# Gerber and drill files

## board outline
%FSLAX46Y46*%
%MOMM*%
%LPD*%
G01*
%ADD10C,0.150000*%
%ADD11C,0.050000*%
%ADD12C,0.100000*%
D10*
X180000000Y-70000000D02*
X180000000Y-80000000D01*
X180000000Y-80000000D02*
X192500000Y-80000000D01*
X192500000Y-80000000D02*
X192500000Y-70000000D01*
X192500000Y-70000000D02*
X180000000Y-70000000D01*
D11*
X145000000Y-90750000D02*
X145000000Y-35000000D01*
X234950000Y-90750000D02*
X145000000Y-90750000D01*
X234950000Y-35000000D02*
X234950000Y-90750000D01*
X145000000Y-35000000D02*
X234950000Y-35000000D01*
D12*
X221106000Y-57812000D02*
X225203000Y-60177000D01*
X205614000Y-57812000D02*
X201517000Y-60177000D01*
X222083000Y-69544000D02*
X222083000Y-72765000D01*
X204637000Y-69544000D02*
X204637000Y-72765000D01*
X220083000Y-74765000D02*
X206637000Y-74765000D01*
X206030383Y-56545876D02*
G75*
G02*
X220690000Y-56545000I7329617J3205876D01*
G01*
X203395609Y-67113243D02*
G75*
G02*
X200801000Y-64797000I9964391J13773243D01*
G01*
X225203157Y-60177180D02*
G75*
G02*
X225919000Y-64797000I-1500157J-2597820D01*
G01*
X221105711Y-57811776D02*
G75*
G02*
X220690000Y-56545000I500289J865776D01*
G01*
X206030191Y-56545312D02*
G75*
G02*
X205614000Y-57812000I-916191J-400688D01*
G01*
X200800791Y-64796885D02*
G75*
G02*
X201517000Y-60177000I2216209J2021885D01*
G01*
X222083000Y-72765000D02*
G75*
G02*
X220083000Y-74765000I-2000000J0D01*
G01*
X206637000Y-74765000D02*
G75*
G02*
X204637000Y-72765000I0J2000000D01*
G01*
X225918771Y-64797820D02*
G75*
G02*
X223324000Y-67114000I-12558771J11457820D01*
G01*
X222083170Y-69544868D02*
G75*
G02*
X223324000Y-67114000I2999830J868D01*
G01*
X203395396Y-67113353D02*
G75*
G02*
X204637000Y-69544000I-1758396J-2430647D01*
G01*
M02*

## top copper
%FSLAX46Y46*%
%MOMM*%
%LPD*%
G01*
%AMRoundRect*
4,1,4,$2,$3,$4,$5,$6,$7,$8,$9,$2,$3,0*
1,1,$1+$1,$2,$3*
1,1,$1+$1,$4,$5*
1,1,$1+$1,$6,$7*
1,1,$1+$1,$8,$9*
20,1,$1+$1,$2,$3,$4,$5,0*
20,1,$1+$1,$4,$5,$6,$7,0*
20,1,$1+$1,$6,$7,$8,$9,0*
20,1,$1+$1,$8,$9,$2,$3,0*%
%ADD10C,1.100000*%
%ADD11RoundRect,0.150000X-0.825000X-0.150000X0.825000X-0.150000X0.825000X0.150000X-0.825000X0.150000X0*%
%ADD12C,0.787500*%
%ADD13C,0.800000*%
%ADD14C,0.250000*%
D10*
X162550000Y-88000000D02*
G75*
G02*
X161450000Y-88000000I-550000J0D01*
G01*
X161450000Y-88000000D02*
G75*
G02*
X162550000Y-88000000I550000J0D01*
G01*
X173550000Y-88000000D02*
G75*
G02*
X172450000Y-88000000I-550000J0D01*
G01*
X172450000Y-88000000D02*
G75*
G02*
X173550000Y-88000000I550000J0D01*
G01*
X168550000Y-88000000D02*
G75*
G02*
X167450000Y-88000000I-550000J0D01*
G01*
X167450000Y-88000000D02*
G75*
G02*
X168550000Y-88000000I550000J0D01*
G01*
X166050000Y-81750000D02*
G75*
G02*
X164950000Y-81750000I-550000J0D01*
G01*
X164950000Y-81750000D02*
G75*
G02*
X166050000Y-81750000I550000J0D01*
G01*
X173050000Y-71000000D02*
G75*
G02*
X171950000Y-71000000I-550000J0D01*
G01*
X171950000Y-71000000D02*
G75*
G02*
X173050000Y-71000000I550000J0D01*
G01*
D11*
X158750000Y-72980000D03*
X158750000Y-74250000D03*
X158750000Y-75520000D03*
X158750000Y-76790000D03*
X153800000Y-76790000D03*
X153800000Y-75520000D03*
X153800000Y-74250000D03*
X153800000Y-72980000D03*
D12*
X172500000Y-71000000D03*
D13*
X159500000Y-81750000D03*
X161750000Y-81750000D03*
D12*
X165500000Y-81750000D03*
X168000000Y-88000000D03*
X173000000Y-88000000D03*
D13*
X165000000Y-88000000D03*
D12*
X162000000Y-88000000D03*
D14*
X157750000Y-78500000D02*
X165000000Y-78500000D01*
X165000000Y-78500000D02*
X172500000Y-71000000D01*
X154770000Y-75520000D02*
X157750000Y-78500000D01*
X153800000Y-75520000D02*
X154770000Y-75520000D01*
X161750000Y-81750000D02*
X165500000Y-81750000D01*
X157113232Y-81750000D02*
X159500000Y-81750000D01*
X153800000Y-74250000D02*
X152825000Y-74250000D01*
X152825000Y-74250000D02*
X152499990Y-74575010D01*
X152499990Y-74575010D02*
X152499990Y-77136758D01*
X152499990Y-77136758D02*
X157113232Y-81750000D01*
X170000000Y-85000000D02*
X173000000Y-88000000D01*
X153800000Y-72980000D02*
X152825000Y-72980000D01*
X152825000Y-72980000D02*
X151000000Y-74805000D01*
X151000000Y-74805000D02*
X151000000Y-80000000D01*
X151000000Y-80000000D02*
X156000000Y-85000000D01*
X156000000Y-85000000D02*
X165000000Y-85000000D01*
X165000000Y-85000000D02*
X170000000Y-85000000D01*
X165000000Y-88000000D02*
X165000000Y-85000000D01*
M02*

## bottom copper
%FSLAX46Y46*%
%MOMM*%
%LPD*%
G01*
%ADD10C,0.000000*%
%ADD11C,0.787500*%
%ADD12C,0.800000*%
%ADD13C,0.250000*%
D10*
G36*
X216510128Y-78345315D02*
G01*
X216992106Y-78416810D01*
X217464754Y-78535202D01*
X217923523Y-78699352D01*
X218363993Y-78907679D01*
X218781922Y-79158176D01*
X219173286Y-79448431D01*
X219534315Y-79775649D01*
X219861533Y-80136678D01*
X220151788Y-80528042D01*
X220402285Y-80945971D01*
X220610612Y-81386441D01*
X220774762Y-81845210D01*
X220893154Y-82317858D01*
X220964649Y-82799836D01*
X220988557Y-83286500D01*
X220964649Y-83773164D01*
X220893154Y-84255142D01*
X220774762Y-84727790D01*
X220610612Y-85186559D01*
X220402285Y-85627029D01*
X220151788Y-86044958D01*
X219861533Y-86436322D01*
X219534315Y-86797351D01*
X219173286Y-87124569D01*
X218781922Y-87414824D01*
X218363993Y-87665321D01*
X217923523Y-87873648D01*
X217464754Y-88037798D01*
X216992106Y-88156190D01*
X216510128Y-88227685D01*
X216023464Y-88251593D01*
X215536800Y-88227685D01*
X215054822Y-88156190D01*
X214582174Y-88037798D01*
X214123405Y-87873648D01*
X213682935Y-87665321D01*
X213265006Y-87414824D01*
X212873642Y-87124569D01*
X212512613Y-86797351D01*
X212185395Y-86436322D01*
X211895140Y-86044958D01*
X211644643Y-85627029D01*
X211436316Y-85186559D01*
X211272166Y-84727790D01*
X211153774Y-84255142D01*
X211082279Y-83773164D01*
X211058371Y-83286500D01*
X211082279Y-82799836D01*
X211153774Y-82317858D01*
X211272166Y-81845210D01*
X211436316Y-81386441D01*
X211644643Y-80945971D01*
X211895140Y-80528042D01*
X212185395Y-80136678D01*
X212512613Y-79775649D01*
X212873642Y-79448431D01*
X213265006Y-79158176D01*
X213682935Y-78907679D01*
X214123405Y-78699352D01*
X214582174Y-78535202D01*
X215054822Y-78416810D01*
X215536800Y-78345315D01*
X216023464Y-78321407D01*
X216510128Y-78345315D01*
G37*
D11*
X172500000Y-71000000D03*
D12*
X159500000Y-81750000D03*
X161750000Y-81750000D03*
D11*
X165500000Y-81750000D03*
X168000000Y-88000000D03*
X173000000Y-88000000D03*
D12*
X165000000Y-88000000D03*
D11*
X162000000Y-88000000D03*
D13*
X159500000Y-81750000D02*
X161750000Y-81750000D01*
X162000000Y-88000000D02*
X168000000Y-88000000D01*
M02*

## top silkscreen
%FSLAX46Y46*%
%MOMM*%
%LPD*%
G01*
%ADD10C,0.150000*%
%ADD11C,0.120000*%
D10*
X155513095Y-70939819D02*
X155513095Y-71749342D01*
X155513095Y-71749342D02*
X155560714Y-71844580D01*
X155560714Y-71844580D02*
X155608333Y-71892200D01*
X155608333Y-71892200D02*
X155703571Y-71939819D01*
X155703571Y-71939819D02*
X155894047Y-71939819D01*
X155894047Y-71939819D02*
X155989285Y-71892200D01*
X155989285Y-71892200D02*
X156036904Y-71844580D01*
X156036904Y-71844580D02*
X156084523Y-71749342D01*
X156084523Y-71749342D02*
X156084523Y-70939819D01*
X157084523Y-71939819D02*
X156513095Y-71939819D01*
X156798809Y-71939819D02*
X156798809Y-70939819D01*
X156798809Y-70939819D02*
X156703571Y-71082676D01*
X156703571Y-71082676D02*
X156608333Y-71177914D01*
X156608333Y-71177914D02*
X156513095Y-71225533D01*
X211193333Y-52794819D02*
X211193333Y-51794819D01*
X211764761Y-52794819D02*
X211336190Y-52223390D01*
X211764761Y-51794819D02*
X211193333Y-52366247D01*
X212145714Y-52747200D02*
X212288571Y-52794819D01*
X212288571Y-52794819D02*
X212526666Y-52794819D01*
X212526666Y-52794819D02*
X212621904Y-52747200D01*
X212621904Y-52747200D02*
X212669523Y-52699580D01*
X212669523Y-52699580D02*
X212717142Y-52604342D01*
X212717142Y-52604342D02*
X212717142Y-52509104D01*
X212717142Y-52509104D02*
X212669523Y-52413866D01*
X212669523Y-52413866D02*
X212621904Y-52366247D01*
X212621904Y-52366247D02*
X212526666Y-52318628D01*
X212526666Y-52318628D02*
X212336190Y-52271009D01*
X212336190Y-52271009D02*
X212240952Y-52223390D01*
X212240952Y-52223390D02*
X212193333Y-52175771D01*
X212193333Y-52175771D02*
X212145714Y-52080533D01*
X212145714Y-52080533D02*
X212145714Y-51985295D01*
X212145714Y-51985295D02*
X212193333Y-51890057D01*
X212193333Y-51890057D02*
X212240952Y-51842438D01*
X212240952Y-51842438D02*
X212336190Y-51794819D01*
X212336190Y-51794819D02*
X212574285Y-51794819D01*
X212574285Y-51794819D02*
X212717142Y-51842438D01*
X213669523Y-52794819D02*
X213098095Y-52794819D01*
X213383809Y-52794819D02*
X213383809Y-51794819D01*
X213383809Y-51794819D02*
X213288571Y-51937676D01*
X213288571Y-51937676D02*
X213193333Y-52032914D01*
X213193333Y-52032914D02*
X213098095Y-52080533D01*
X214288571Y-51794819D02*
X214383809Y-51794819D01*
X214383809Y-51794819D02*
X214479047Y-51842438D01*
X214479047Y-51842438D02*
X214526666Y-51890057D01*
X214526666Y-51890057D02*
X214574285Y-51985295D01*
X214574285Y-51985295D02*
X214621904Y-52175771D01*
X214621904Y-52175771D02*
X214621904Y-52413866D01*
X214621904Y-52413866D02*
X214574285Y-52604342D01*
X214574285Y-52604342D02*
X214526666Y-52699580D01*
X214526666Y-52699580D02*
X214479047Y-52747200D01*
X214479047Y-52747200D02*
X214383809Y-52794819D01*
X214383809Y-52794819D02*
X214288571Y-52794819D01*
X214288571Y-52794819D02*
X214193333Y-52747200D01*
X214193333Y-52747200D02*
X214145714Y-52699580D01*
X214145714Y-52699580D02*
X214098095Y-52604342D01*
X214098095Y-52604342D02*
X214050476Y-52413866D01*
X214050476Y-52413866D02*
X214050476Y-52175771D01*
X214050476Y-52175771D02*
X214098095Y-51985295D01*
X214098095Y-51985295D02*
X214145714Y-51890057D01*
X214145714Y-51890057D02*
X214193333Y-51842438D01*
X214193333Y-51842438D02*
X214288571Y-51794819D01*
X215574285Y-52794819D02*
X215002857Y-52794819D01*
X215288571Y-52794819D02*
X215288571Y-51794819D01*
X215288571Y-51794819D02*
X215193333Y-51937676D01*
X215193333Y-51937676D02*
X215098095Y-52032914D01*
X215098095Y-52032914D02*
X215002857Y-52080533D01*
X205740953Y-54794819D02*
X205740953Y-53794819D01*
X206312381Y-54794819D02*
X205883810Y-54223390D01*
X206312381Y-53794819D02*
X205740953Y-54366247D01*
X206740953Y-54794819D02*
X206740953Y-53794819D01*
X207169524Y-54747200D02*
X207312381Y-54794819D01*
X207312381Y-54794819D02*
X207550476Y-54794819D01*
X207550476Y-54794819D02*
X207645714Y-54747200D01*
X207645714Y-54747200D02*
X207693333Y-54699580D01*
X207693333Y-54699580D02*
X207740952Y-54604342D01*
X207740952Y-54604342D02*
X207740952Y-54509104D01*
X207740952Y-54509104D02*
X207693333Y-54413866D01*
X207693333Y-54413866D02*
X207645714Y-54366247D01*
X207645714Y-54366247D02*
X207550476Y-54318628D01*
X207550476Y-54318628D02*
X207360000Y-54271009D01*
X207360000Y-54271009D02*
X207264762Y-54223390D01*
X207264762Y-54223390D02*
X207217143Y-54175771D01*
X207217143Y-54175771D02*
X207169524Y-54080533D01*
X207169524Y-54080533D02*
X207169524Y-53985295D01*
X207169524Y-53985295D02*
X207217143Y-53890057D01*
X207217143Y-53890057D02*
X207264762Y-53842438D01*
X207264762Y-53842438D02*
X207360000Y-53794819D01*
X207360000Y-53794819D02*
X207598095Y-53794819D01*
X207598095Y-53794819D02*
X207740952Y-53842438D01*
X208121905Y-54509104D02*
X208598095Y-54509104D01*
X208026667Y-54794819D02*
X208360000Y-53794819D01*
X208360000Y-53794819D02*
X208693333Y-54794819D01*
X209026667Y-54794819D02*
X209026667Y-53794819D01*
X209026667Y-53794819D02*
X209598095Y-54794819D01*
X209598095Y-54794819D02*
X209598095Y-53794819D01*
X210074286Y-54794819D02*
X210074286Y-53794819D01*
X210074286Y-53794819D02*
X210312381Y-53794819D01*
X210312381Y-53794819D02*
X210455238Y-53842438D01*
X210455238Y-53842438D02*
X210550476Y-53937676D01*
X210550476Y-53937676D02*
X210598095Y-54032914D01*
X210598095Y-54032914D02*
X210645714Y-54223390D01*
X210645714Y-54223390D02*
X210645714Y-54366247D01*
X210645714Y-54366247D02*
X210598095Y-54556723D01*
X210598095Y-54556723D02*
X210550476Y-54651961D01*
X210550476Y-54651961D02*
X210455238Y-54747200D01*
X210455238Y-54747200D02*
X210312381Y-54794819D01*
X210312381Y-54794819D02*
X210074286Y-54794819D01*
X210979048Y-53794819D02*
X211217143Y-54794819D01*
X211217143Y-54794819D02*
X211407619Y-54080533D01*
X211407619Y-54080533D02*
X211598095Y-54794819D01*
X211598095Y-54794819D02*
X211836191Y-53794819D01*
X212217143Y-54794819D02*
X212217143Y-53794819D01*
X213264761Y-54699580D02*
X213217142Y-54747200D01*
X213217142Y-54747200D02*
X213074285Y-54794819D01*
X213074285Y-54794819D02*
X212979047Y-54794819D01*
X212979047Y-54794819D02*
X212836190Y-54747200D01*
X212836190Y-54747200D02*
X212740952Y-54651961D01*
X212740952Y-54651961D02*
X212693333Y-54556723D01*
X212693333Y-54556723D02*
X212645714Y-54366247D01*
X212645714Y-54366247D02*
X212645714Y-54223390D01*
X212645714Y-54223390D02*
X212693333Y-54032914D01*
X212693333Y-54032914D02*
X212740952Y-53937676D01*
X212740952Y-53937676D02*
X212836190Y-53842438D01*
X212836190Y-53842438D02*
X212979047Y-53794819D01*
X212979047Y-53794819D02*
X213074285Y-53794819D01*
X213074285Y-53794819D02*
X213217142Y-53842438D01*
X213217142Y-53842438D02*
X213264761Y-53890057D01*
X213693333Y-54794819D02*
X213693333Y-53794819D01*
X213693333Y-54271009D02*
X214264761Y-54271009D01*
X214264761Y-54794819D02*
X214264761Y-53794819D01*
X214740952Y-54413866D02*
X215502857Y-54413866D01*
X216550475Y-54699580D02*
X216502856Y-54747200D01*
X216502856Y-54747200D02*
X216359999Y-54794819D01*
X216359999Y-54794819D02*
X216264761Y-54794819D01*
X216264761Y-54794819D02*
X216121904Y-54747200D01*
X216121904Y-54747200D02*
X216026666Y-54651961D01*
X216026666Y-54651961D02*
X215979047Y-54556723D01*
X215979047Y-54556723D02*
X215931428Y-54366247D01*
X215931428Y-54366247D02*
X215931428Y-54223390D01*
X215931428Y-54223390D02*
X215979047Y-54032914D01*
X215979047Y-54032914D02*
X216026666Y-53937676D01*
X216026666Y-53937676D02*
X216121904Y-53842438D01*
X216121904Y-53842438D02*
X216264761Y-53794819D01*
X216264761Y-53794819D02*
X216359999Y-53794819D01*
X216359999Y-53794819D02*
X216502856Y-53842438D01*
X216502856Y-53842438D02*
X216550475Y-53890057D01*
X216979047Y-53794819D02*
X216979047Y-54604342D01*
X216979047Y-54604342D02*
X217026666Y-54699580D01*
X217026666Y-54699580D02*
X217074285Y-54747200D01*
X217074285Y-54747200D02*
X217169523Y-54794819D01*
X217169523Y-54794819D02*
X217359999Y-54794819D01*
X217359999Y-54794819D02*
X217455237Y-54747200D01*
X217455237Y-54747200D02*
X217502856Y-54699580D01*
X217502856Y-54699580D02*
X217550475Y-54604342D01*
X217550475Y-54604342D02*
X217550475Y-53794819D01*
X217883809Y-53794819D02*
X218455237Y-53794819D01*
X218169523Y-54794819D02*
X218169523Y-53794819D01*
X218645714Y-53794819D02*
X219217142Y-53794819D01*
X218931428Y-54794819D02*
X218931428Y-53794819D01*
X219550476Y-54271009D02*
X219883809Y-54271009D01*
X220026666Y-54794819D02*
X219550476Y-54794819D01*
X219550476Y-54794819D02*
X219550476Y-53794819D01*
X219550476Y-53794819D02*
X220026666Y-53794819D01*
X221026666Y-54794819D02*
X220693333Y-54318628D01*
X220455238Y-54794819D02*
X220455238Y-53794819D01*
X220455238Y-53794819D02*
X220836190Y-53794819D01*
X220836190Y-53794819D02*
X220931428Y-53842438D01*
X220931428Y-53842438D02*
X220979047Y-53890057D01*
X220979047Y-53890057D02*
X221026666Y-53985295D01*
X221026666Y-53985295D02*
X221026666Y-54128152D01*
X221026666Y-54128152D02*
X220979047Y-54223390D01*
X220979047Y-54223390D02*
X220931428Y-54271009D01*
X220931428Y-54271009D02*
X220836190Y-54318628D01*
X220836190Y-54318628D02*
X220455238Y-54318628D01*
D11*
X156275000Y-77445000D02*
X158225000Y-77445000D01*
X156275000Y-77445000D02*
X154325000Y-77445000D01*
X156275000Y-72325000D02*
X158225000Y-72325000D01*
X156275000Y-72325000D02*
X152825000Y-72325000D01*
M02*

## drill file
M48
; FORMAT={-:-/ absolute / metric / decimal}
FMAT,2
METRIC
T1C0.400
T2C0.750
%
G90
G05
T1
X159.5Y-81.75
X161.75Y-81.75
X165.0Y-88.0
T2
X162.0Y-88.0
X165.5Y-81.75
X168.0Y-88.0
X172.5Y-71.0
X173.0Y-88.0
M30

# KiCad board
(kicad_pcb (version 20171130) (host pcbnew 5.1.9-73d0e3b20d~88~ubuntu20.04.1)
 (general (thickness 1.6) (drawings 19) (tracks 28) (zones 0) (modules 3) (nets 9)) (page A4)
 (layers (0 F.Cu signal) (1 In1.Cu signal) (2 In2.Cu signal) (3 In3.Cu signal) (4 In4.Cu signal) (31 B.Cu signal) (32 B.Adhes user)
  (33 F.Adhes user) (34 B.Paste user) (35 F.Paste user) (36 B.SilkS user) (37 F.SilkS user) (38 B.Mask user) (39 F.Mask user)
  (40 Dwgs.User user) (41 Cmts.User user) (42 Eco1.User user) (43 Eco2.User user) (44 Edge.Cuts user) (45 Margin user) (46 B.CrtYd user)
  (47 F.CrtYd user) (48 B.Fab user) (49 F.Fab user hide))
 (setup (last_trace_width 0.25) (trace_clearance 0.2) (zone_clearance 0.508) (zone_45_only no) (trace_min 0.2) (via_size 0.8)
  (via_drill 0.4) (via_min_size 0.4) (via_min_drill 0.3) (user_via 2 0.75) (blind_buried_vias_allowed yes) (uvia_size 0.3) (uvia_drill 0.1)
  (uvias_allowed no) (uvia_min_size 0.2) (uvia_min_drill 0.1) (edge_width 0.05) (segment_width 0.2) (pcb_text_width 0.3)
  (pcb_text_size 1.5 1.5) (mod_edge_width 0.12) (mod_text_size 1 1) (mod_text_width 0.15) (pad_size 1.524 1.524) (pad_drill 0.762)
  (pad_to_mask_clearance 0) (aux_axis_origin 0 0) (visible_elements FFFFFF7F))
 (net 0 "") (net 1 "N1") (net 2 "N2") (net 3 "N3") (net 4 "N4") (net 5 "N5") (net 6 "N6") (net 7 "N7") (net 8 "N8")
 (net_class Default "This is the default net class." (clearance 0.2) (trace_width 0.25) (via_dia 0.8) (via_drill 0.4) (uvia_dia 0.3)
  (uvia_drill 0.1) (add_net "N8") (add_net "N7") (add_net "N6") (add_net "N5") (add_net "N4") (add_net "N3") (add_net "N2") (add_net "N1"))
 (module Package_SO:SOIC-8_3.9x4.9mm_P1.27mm (layer F.Cu) (at 156.275 74.885)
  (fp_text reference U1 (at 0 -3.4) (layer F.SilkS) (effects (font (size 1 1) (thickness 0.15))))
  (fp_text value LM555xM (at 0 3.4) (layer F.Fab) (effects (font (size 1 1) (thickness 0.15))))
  (fp_line (start 0 2.56) (end 1.95 2.56) (layer F.SilkS) (width 0.12))
  (fp_line (start 0 2.56) (end -1.95 2.56) (layer F.SilkS) (width 0.12))
  (fp_line (start 0 -2.56) (end 1.95 -2.56) (layer F.SilkS) (width 0.12))
  (fp_line (start 0 -2.56) (end -3.45 -2.56) (layer F.SilkS) (width 0.12))
  (pad 8 smd roundrect (at 2.475 -1.905) (size 1.95 0.6) (layers F.Cu F.Paste F.Mask) (roundrect_rratio 0.25) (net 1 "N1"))
  (pad 7 smd roundrect (at 2.475 -0.635) (size 1.95 0.6) (layers F.Cu F.Paste F.Mask) (roundrect_rratio 0.25) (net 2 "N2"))
  (pad 6 smd roundrect (at 2.475 0.635) (size 1.95 0.6) (layers F.Cu F.Paste F.Mask) (roundrect_rratio 0.25) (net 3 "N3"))
  (pad 5 smd roundrect (at 2.475 1.905) (size 1.95 0.6) (layers F.Cu F.Paste F.Mask) (roundrect_rratio 0.25) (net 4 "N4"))
  (pad 4 smd roundrect (at -2.475 1.905) (size 1.95 0.6) (layers F.Cu F.Paste F.Mask) (roundrect_rratio 0.25) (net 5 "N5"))
  (pad 3 smd roundrect (at -2.475 0.635) (size 1.95 0.6) (layers F.Cu F.Paste F.Mask) (roundrect_rratio 0.25) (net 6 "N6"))
  (pad 2 smd roundrect (at -2.475 -0.635) (size 1.95 0.6) (layers F.Cu F.Paste F.Mask) (roundrect_rratio 0.25) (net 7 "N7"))
  (pad 1 smd roundrect (at -2.475 -1.905) (size 1.95 0.6) (layers F.Cu F.Paste F.Mask) (roundrect_rratio 0.25) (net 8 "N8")))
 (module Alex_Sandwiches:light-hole (layer F.Cu) (at 201.93 77.47)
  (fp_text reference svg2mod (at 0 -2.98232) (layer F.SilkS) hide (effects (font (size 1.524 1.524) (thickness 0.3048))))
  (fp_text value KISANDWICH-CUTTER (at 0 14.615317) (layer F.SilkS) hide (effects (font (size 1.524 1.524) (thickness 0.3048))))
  (fp_poly
   (pts (xy 19.058557 5.8165) (xy 19.034649 6.303164) (xy 18.963154 6.785142) (xy 18.844762 7.25779) (xy 18.680612 7.716559)
    (xy 18.472285 8.157029) (xy 18.221788 8.574958) (xy 17.931533 8.966322) (xy 17.604315 9.327351) (xy 17.243286 9.654569)
    (xy 16.851922 9.944824) (xy 16.433993 10.195321) (xy 15.993523 10.403648) (xy 15.534754 10.567798) (xy 15.062106 10.68619)
    (xy 14.580128 10.757685) (xy 14.093464 10.781593) (xy 13.6068 10.757685) (xy 13.124822 10.68619) (xy 12.652174 10.567798)
    (xy 12.193405 10.403648) (xy 11.752935 10.195321) (xy 11.335006 9.944824) (xy 10.943642 9.654569) (xy 10.582613 9.327351)
    (xy 10.255395 8.966322) (xy 9.96514 8.574958) (xy 9.714643 8.157029) (xy 9.506316 7.716559) (xy 9.342166 7.25779) (xy 9.223774 6.785142)
    (xy 9.152279 6.303164) (xy 9.128371 5.8165) (xy 9.152279 5.329836) (xy 9.223774 4.847858) (xy 9.342166 4.37521) (xy 9.506316 3.916441)
    (xy 9.714643 3.475971) (xy 9.96514 3.058042) (xy 10.255395 2.666678) (xy 10.582613 2.305649) (xy 10.943642 1.978431)
    (xy 11.335006 1.688176) (xy 11.752935 1.437679) (xy 12.193405 1.229352) (xy 12.652174 1.065202) (xy 13.124822 0.94681)
    (xy 13.6068 0.875315) (xy 14.093464 0.851407) (xy 14.580128 0.875315) (xy 15.062106 0.94681) (xy 15.534754 1.065202)
    (xy 15.993523 1.229352) (xy 16.433993 1.437679) (xy 16.851922 1.688176) (xy 17.243286 1.978431) (xy 17.604315 2.305649)
    (xy 17.931533 2.666678) (xy 18.221788 3.058042) (xy 18.472285 3.475971) (xy 18.680612 3.916441) (xy 18.844762 4.37521)
    (xy 18.963154 4.847858) (xy 19.034649 5.329836) (xy 19.058557 5.8165))
   (layer B.Cu) (width 0)))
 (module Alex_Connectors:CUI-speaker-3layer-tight (layer F.Cu) (at 213.36 53.34 180)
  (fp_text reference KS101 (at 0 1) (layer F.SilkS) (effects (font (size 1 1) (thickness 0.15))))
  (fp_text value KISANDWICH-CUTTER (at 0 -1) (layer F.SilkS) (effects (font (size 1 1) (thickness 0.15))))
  (fp_line (start -7.746 -4.472) (end -11.843 -6.837) (layer Edge.Cuts) (width 0.1))
  (fp_line (start 7.746 -4.472) (end 11.843 -6.837) (layer Edge.Cuts) (width 0.1))
  (fp_line (start -8.723 -16.204) (end -8.723 -19.425) (layer Edge.Cuts) (width 0.1))
  (fp_line (start 8.723 -16.204) (end 8.723 -19.425) (layer Edge.Cuts) (width 0.1))
  (fp_line (start -6.723 -21.425) (end 6.723 -21.425) (layer Edge.Cuts) (width 0.1))
  (fp_arc (start 0 0) (end -7.33 -3.205) (angle -227.241) (layer Edge.Cuts) (width 0.1))
  (fp_arc (start 0 0) (end 12.559 -11.457) (angle -11.743) (layer Edge.Cuts) (width 0.1))
  (fp_arc (start -10.343 -9.435) (end -12.559 -11.457) (angle -102.374) (layer Edge.Cuts) (width 0.1))
  (fp_arc (start -8.246 -3.606) (end -7.33 -3.205) (angle -83.621) (layer Edge.Cuts) (width 0.1))
  (fp_arc (start 8.246 -3.606) (end 7.746 -4.472) (angle -83.621) (layer Edge.Cuts) (width 0.1))
  (fp_arc (start 10.343 -9.435) (end 11.843 -6.837) (angle -102.374) (layer Edge.Cuts) (width 0.1))
  (fp_arc (start -6.723 -19.425) (end -6.723 -21.425) (angle -90) (layer Edge.Cuts) (width 0.1))
  (fp_arc (start 6.723 -19.425) (end 8.723 -19.425) (angle -90) (layer Edge.Cuts) (width 0.1))
  (fp_arc (start 0 0) (end -9.964 -13.774) (angle -11.743) (layer Edge.Cuts) (width 0.1))
  (fp_arc (start -11.723 -16.204) (end -9.964 -13.774) (angle -54.117) (layer Edge.Cuts) (width 0.1))
  (fp_arc (start 11.723 -16.204) (end 8.723 -16.204) (angle -54.117) (layer Edge.Cuts) (width 0.1)))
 (gr_circle (center 162 88) (end 162 88.55) (layer F.Cu) (width 1.1))
 (gr_circle (center 173 88) (end 173 88.55) (layer F.Cu) (width 1.1))
 (gr_circle (center 168 88) (end 168 88.55) (layer F.Cu) (width 1.1))
 (gr_circle (center 165.5 81.75) (end 165.5 82.3) (layer F.Cu) (width 1.1))
 (gr_circle (center 172.5 71) (end 172.5 71.55) (layer F.Cu) (width 1.1))
 (gr_line (start 180 70) (end 180 80) (layer Edge.Cuts) (width 0.15))
 (gr_line (start 180 80) (end 192.5 80) (layer Edge.Cuts) (width 0.15))
 (gr_line (start 192.5 80) (end 192.5 70) (layer Edge.Cuts) (width 0.15))
 (gr_line (start 192.5 70) (end 180 70) (layer Edge.Cuts) (width 0.15))
 (gr_line (start 145 90.75) (end 145 35) (layer Edge.Cuts) (width 0.05))
 (gr_line (start 234.95 90.75) (end 145 90.75) (layer Edge.Cuts) (width 0.05))
 (gr_line (start 234.95 35) (end 234.95 90.75) (layer Edge.Cuts) (width 0.05))
 (gr_line (start 145 35) (end 234.95 35) (layer Edge.Cuts) (width 0.05))
 (via (at 172.5 71) (size 0.7875) (drill 0.75) (layers F.Cu B.Cu) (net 6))
 (segment (start 157.75 78.5) (end 165 78.5) (width 0.25) (layer F.Cu) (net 6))
 (segment (start 165 78.5) (end 172.5 71) (width 0.25) (layer F.Cu) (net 6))
 (segment (start 154.77 75.52) (end 157.75 78.5) (width 0.25) (layer F.Cu) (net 6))
 (segment (start 153.8 75.52) (end 154.77 75.52) (width 0.25) (layer F.Cu) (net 6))
 (via (at 159.5 81.75) (size 0.8) (drill 0.4) (layers F.Cu B.Cu) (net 7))
 (via (at 161.75 81.75) (size 0.8) (drill 0.4) (layers F.Cu B.Cu) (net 7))
 (via (at 165.5 81.75) (size 0.7875) (drill 0.75) (layers F.Cu B.Cu) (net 7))
 (segment (start 161.75 81.75) (end 165.5 81.75) (width 0.25) (layer F.Cu) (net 7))
 (segment (start 159.5 81.75) (end 161.75 81.75) (width 0.25) (layer B.Cu) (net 7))
 (segment (start 157.113232 81.75) (end 159.5 81.75) (width 0.25) (layer F.Cu) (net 7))
 (segment (start 153.8 74.25) (end 152.825 74.25) (width 0.25) (layer F.Cu) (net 7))
 (segment (start 152.825 74.25) (end 152.49999 74.57501) (width 0.25) (layer F.Cu) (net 7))
 (segment (start 152.49999 74.57501) (end 152.49999 77.136758) (width 0.25) (layer F.Cu) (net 7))
 (segment (start 152.49999 77.136758) (end 157.113232 81.75) (width 0.25) (layer F.Cu) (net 7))
 (via (at 168 88) (size 0.7875) (drill 0.75) (layers F.Cu B.Cu) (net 8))
 (via (at 173 88) (size 0.7875) (drill 0.75) (layers F.Cu B.Cu) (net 8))
 (via (at 165 88) (size 0.8) (drill 0.4) (layers F.Cu B.Cu) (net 8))
 (via (at 162 88) (size 0.7875) (drill 0.75) (layers F.Cu B.Cu) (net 8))
 (segment (start 162 88) (end 168 88) (width 0.25) (layer B.Cu) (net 8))
 (segment (start 170 85) (end 173 88) (width 0.25) (layer F.Cu) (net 8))
 (segment (start 153.8 72.98) (end 152.825 72.98) (width 0.25) (layer F.Cu) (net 8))
 (segment (start 152.825 72.98) (end 151 74.805) (width 0.25) (layer F.Cu) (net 8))
 (segment (start 151 74.805) (end 151 80) (width 0.25) (layer F.Cu) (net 8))
 (segment (start 151 80) (end 156 85) (width 0.25) (layer F.Cu) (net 8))
 (segment (start 156 85) (end 165 85) (width 0.25) (layer F.Cu) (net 8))
 (segment (start 165 85) (end 170 85) (width 0.25) (layer F.Cu) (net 8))
 (segment (start 165 88) (end 165 85) (width 0.25) (layer F.Cu) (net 8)))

